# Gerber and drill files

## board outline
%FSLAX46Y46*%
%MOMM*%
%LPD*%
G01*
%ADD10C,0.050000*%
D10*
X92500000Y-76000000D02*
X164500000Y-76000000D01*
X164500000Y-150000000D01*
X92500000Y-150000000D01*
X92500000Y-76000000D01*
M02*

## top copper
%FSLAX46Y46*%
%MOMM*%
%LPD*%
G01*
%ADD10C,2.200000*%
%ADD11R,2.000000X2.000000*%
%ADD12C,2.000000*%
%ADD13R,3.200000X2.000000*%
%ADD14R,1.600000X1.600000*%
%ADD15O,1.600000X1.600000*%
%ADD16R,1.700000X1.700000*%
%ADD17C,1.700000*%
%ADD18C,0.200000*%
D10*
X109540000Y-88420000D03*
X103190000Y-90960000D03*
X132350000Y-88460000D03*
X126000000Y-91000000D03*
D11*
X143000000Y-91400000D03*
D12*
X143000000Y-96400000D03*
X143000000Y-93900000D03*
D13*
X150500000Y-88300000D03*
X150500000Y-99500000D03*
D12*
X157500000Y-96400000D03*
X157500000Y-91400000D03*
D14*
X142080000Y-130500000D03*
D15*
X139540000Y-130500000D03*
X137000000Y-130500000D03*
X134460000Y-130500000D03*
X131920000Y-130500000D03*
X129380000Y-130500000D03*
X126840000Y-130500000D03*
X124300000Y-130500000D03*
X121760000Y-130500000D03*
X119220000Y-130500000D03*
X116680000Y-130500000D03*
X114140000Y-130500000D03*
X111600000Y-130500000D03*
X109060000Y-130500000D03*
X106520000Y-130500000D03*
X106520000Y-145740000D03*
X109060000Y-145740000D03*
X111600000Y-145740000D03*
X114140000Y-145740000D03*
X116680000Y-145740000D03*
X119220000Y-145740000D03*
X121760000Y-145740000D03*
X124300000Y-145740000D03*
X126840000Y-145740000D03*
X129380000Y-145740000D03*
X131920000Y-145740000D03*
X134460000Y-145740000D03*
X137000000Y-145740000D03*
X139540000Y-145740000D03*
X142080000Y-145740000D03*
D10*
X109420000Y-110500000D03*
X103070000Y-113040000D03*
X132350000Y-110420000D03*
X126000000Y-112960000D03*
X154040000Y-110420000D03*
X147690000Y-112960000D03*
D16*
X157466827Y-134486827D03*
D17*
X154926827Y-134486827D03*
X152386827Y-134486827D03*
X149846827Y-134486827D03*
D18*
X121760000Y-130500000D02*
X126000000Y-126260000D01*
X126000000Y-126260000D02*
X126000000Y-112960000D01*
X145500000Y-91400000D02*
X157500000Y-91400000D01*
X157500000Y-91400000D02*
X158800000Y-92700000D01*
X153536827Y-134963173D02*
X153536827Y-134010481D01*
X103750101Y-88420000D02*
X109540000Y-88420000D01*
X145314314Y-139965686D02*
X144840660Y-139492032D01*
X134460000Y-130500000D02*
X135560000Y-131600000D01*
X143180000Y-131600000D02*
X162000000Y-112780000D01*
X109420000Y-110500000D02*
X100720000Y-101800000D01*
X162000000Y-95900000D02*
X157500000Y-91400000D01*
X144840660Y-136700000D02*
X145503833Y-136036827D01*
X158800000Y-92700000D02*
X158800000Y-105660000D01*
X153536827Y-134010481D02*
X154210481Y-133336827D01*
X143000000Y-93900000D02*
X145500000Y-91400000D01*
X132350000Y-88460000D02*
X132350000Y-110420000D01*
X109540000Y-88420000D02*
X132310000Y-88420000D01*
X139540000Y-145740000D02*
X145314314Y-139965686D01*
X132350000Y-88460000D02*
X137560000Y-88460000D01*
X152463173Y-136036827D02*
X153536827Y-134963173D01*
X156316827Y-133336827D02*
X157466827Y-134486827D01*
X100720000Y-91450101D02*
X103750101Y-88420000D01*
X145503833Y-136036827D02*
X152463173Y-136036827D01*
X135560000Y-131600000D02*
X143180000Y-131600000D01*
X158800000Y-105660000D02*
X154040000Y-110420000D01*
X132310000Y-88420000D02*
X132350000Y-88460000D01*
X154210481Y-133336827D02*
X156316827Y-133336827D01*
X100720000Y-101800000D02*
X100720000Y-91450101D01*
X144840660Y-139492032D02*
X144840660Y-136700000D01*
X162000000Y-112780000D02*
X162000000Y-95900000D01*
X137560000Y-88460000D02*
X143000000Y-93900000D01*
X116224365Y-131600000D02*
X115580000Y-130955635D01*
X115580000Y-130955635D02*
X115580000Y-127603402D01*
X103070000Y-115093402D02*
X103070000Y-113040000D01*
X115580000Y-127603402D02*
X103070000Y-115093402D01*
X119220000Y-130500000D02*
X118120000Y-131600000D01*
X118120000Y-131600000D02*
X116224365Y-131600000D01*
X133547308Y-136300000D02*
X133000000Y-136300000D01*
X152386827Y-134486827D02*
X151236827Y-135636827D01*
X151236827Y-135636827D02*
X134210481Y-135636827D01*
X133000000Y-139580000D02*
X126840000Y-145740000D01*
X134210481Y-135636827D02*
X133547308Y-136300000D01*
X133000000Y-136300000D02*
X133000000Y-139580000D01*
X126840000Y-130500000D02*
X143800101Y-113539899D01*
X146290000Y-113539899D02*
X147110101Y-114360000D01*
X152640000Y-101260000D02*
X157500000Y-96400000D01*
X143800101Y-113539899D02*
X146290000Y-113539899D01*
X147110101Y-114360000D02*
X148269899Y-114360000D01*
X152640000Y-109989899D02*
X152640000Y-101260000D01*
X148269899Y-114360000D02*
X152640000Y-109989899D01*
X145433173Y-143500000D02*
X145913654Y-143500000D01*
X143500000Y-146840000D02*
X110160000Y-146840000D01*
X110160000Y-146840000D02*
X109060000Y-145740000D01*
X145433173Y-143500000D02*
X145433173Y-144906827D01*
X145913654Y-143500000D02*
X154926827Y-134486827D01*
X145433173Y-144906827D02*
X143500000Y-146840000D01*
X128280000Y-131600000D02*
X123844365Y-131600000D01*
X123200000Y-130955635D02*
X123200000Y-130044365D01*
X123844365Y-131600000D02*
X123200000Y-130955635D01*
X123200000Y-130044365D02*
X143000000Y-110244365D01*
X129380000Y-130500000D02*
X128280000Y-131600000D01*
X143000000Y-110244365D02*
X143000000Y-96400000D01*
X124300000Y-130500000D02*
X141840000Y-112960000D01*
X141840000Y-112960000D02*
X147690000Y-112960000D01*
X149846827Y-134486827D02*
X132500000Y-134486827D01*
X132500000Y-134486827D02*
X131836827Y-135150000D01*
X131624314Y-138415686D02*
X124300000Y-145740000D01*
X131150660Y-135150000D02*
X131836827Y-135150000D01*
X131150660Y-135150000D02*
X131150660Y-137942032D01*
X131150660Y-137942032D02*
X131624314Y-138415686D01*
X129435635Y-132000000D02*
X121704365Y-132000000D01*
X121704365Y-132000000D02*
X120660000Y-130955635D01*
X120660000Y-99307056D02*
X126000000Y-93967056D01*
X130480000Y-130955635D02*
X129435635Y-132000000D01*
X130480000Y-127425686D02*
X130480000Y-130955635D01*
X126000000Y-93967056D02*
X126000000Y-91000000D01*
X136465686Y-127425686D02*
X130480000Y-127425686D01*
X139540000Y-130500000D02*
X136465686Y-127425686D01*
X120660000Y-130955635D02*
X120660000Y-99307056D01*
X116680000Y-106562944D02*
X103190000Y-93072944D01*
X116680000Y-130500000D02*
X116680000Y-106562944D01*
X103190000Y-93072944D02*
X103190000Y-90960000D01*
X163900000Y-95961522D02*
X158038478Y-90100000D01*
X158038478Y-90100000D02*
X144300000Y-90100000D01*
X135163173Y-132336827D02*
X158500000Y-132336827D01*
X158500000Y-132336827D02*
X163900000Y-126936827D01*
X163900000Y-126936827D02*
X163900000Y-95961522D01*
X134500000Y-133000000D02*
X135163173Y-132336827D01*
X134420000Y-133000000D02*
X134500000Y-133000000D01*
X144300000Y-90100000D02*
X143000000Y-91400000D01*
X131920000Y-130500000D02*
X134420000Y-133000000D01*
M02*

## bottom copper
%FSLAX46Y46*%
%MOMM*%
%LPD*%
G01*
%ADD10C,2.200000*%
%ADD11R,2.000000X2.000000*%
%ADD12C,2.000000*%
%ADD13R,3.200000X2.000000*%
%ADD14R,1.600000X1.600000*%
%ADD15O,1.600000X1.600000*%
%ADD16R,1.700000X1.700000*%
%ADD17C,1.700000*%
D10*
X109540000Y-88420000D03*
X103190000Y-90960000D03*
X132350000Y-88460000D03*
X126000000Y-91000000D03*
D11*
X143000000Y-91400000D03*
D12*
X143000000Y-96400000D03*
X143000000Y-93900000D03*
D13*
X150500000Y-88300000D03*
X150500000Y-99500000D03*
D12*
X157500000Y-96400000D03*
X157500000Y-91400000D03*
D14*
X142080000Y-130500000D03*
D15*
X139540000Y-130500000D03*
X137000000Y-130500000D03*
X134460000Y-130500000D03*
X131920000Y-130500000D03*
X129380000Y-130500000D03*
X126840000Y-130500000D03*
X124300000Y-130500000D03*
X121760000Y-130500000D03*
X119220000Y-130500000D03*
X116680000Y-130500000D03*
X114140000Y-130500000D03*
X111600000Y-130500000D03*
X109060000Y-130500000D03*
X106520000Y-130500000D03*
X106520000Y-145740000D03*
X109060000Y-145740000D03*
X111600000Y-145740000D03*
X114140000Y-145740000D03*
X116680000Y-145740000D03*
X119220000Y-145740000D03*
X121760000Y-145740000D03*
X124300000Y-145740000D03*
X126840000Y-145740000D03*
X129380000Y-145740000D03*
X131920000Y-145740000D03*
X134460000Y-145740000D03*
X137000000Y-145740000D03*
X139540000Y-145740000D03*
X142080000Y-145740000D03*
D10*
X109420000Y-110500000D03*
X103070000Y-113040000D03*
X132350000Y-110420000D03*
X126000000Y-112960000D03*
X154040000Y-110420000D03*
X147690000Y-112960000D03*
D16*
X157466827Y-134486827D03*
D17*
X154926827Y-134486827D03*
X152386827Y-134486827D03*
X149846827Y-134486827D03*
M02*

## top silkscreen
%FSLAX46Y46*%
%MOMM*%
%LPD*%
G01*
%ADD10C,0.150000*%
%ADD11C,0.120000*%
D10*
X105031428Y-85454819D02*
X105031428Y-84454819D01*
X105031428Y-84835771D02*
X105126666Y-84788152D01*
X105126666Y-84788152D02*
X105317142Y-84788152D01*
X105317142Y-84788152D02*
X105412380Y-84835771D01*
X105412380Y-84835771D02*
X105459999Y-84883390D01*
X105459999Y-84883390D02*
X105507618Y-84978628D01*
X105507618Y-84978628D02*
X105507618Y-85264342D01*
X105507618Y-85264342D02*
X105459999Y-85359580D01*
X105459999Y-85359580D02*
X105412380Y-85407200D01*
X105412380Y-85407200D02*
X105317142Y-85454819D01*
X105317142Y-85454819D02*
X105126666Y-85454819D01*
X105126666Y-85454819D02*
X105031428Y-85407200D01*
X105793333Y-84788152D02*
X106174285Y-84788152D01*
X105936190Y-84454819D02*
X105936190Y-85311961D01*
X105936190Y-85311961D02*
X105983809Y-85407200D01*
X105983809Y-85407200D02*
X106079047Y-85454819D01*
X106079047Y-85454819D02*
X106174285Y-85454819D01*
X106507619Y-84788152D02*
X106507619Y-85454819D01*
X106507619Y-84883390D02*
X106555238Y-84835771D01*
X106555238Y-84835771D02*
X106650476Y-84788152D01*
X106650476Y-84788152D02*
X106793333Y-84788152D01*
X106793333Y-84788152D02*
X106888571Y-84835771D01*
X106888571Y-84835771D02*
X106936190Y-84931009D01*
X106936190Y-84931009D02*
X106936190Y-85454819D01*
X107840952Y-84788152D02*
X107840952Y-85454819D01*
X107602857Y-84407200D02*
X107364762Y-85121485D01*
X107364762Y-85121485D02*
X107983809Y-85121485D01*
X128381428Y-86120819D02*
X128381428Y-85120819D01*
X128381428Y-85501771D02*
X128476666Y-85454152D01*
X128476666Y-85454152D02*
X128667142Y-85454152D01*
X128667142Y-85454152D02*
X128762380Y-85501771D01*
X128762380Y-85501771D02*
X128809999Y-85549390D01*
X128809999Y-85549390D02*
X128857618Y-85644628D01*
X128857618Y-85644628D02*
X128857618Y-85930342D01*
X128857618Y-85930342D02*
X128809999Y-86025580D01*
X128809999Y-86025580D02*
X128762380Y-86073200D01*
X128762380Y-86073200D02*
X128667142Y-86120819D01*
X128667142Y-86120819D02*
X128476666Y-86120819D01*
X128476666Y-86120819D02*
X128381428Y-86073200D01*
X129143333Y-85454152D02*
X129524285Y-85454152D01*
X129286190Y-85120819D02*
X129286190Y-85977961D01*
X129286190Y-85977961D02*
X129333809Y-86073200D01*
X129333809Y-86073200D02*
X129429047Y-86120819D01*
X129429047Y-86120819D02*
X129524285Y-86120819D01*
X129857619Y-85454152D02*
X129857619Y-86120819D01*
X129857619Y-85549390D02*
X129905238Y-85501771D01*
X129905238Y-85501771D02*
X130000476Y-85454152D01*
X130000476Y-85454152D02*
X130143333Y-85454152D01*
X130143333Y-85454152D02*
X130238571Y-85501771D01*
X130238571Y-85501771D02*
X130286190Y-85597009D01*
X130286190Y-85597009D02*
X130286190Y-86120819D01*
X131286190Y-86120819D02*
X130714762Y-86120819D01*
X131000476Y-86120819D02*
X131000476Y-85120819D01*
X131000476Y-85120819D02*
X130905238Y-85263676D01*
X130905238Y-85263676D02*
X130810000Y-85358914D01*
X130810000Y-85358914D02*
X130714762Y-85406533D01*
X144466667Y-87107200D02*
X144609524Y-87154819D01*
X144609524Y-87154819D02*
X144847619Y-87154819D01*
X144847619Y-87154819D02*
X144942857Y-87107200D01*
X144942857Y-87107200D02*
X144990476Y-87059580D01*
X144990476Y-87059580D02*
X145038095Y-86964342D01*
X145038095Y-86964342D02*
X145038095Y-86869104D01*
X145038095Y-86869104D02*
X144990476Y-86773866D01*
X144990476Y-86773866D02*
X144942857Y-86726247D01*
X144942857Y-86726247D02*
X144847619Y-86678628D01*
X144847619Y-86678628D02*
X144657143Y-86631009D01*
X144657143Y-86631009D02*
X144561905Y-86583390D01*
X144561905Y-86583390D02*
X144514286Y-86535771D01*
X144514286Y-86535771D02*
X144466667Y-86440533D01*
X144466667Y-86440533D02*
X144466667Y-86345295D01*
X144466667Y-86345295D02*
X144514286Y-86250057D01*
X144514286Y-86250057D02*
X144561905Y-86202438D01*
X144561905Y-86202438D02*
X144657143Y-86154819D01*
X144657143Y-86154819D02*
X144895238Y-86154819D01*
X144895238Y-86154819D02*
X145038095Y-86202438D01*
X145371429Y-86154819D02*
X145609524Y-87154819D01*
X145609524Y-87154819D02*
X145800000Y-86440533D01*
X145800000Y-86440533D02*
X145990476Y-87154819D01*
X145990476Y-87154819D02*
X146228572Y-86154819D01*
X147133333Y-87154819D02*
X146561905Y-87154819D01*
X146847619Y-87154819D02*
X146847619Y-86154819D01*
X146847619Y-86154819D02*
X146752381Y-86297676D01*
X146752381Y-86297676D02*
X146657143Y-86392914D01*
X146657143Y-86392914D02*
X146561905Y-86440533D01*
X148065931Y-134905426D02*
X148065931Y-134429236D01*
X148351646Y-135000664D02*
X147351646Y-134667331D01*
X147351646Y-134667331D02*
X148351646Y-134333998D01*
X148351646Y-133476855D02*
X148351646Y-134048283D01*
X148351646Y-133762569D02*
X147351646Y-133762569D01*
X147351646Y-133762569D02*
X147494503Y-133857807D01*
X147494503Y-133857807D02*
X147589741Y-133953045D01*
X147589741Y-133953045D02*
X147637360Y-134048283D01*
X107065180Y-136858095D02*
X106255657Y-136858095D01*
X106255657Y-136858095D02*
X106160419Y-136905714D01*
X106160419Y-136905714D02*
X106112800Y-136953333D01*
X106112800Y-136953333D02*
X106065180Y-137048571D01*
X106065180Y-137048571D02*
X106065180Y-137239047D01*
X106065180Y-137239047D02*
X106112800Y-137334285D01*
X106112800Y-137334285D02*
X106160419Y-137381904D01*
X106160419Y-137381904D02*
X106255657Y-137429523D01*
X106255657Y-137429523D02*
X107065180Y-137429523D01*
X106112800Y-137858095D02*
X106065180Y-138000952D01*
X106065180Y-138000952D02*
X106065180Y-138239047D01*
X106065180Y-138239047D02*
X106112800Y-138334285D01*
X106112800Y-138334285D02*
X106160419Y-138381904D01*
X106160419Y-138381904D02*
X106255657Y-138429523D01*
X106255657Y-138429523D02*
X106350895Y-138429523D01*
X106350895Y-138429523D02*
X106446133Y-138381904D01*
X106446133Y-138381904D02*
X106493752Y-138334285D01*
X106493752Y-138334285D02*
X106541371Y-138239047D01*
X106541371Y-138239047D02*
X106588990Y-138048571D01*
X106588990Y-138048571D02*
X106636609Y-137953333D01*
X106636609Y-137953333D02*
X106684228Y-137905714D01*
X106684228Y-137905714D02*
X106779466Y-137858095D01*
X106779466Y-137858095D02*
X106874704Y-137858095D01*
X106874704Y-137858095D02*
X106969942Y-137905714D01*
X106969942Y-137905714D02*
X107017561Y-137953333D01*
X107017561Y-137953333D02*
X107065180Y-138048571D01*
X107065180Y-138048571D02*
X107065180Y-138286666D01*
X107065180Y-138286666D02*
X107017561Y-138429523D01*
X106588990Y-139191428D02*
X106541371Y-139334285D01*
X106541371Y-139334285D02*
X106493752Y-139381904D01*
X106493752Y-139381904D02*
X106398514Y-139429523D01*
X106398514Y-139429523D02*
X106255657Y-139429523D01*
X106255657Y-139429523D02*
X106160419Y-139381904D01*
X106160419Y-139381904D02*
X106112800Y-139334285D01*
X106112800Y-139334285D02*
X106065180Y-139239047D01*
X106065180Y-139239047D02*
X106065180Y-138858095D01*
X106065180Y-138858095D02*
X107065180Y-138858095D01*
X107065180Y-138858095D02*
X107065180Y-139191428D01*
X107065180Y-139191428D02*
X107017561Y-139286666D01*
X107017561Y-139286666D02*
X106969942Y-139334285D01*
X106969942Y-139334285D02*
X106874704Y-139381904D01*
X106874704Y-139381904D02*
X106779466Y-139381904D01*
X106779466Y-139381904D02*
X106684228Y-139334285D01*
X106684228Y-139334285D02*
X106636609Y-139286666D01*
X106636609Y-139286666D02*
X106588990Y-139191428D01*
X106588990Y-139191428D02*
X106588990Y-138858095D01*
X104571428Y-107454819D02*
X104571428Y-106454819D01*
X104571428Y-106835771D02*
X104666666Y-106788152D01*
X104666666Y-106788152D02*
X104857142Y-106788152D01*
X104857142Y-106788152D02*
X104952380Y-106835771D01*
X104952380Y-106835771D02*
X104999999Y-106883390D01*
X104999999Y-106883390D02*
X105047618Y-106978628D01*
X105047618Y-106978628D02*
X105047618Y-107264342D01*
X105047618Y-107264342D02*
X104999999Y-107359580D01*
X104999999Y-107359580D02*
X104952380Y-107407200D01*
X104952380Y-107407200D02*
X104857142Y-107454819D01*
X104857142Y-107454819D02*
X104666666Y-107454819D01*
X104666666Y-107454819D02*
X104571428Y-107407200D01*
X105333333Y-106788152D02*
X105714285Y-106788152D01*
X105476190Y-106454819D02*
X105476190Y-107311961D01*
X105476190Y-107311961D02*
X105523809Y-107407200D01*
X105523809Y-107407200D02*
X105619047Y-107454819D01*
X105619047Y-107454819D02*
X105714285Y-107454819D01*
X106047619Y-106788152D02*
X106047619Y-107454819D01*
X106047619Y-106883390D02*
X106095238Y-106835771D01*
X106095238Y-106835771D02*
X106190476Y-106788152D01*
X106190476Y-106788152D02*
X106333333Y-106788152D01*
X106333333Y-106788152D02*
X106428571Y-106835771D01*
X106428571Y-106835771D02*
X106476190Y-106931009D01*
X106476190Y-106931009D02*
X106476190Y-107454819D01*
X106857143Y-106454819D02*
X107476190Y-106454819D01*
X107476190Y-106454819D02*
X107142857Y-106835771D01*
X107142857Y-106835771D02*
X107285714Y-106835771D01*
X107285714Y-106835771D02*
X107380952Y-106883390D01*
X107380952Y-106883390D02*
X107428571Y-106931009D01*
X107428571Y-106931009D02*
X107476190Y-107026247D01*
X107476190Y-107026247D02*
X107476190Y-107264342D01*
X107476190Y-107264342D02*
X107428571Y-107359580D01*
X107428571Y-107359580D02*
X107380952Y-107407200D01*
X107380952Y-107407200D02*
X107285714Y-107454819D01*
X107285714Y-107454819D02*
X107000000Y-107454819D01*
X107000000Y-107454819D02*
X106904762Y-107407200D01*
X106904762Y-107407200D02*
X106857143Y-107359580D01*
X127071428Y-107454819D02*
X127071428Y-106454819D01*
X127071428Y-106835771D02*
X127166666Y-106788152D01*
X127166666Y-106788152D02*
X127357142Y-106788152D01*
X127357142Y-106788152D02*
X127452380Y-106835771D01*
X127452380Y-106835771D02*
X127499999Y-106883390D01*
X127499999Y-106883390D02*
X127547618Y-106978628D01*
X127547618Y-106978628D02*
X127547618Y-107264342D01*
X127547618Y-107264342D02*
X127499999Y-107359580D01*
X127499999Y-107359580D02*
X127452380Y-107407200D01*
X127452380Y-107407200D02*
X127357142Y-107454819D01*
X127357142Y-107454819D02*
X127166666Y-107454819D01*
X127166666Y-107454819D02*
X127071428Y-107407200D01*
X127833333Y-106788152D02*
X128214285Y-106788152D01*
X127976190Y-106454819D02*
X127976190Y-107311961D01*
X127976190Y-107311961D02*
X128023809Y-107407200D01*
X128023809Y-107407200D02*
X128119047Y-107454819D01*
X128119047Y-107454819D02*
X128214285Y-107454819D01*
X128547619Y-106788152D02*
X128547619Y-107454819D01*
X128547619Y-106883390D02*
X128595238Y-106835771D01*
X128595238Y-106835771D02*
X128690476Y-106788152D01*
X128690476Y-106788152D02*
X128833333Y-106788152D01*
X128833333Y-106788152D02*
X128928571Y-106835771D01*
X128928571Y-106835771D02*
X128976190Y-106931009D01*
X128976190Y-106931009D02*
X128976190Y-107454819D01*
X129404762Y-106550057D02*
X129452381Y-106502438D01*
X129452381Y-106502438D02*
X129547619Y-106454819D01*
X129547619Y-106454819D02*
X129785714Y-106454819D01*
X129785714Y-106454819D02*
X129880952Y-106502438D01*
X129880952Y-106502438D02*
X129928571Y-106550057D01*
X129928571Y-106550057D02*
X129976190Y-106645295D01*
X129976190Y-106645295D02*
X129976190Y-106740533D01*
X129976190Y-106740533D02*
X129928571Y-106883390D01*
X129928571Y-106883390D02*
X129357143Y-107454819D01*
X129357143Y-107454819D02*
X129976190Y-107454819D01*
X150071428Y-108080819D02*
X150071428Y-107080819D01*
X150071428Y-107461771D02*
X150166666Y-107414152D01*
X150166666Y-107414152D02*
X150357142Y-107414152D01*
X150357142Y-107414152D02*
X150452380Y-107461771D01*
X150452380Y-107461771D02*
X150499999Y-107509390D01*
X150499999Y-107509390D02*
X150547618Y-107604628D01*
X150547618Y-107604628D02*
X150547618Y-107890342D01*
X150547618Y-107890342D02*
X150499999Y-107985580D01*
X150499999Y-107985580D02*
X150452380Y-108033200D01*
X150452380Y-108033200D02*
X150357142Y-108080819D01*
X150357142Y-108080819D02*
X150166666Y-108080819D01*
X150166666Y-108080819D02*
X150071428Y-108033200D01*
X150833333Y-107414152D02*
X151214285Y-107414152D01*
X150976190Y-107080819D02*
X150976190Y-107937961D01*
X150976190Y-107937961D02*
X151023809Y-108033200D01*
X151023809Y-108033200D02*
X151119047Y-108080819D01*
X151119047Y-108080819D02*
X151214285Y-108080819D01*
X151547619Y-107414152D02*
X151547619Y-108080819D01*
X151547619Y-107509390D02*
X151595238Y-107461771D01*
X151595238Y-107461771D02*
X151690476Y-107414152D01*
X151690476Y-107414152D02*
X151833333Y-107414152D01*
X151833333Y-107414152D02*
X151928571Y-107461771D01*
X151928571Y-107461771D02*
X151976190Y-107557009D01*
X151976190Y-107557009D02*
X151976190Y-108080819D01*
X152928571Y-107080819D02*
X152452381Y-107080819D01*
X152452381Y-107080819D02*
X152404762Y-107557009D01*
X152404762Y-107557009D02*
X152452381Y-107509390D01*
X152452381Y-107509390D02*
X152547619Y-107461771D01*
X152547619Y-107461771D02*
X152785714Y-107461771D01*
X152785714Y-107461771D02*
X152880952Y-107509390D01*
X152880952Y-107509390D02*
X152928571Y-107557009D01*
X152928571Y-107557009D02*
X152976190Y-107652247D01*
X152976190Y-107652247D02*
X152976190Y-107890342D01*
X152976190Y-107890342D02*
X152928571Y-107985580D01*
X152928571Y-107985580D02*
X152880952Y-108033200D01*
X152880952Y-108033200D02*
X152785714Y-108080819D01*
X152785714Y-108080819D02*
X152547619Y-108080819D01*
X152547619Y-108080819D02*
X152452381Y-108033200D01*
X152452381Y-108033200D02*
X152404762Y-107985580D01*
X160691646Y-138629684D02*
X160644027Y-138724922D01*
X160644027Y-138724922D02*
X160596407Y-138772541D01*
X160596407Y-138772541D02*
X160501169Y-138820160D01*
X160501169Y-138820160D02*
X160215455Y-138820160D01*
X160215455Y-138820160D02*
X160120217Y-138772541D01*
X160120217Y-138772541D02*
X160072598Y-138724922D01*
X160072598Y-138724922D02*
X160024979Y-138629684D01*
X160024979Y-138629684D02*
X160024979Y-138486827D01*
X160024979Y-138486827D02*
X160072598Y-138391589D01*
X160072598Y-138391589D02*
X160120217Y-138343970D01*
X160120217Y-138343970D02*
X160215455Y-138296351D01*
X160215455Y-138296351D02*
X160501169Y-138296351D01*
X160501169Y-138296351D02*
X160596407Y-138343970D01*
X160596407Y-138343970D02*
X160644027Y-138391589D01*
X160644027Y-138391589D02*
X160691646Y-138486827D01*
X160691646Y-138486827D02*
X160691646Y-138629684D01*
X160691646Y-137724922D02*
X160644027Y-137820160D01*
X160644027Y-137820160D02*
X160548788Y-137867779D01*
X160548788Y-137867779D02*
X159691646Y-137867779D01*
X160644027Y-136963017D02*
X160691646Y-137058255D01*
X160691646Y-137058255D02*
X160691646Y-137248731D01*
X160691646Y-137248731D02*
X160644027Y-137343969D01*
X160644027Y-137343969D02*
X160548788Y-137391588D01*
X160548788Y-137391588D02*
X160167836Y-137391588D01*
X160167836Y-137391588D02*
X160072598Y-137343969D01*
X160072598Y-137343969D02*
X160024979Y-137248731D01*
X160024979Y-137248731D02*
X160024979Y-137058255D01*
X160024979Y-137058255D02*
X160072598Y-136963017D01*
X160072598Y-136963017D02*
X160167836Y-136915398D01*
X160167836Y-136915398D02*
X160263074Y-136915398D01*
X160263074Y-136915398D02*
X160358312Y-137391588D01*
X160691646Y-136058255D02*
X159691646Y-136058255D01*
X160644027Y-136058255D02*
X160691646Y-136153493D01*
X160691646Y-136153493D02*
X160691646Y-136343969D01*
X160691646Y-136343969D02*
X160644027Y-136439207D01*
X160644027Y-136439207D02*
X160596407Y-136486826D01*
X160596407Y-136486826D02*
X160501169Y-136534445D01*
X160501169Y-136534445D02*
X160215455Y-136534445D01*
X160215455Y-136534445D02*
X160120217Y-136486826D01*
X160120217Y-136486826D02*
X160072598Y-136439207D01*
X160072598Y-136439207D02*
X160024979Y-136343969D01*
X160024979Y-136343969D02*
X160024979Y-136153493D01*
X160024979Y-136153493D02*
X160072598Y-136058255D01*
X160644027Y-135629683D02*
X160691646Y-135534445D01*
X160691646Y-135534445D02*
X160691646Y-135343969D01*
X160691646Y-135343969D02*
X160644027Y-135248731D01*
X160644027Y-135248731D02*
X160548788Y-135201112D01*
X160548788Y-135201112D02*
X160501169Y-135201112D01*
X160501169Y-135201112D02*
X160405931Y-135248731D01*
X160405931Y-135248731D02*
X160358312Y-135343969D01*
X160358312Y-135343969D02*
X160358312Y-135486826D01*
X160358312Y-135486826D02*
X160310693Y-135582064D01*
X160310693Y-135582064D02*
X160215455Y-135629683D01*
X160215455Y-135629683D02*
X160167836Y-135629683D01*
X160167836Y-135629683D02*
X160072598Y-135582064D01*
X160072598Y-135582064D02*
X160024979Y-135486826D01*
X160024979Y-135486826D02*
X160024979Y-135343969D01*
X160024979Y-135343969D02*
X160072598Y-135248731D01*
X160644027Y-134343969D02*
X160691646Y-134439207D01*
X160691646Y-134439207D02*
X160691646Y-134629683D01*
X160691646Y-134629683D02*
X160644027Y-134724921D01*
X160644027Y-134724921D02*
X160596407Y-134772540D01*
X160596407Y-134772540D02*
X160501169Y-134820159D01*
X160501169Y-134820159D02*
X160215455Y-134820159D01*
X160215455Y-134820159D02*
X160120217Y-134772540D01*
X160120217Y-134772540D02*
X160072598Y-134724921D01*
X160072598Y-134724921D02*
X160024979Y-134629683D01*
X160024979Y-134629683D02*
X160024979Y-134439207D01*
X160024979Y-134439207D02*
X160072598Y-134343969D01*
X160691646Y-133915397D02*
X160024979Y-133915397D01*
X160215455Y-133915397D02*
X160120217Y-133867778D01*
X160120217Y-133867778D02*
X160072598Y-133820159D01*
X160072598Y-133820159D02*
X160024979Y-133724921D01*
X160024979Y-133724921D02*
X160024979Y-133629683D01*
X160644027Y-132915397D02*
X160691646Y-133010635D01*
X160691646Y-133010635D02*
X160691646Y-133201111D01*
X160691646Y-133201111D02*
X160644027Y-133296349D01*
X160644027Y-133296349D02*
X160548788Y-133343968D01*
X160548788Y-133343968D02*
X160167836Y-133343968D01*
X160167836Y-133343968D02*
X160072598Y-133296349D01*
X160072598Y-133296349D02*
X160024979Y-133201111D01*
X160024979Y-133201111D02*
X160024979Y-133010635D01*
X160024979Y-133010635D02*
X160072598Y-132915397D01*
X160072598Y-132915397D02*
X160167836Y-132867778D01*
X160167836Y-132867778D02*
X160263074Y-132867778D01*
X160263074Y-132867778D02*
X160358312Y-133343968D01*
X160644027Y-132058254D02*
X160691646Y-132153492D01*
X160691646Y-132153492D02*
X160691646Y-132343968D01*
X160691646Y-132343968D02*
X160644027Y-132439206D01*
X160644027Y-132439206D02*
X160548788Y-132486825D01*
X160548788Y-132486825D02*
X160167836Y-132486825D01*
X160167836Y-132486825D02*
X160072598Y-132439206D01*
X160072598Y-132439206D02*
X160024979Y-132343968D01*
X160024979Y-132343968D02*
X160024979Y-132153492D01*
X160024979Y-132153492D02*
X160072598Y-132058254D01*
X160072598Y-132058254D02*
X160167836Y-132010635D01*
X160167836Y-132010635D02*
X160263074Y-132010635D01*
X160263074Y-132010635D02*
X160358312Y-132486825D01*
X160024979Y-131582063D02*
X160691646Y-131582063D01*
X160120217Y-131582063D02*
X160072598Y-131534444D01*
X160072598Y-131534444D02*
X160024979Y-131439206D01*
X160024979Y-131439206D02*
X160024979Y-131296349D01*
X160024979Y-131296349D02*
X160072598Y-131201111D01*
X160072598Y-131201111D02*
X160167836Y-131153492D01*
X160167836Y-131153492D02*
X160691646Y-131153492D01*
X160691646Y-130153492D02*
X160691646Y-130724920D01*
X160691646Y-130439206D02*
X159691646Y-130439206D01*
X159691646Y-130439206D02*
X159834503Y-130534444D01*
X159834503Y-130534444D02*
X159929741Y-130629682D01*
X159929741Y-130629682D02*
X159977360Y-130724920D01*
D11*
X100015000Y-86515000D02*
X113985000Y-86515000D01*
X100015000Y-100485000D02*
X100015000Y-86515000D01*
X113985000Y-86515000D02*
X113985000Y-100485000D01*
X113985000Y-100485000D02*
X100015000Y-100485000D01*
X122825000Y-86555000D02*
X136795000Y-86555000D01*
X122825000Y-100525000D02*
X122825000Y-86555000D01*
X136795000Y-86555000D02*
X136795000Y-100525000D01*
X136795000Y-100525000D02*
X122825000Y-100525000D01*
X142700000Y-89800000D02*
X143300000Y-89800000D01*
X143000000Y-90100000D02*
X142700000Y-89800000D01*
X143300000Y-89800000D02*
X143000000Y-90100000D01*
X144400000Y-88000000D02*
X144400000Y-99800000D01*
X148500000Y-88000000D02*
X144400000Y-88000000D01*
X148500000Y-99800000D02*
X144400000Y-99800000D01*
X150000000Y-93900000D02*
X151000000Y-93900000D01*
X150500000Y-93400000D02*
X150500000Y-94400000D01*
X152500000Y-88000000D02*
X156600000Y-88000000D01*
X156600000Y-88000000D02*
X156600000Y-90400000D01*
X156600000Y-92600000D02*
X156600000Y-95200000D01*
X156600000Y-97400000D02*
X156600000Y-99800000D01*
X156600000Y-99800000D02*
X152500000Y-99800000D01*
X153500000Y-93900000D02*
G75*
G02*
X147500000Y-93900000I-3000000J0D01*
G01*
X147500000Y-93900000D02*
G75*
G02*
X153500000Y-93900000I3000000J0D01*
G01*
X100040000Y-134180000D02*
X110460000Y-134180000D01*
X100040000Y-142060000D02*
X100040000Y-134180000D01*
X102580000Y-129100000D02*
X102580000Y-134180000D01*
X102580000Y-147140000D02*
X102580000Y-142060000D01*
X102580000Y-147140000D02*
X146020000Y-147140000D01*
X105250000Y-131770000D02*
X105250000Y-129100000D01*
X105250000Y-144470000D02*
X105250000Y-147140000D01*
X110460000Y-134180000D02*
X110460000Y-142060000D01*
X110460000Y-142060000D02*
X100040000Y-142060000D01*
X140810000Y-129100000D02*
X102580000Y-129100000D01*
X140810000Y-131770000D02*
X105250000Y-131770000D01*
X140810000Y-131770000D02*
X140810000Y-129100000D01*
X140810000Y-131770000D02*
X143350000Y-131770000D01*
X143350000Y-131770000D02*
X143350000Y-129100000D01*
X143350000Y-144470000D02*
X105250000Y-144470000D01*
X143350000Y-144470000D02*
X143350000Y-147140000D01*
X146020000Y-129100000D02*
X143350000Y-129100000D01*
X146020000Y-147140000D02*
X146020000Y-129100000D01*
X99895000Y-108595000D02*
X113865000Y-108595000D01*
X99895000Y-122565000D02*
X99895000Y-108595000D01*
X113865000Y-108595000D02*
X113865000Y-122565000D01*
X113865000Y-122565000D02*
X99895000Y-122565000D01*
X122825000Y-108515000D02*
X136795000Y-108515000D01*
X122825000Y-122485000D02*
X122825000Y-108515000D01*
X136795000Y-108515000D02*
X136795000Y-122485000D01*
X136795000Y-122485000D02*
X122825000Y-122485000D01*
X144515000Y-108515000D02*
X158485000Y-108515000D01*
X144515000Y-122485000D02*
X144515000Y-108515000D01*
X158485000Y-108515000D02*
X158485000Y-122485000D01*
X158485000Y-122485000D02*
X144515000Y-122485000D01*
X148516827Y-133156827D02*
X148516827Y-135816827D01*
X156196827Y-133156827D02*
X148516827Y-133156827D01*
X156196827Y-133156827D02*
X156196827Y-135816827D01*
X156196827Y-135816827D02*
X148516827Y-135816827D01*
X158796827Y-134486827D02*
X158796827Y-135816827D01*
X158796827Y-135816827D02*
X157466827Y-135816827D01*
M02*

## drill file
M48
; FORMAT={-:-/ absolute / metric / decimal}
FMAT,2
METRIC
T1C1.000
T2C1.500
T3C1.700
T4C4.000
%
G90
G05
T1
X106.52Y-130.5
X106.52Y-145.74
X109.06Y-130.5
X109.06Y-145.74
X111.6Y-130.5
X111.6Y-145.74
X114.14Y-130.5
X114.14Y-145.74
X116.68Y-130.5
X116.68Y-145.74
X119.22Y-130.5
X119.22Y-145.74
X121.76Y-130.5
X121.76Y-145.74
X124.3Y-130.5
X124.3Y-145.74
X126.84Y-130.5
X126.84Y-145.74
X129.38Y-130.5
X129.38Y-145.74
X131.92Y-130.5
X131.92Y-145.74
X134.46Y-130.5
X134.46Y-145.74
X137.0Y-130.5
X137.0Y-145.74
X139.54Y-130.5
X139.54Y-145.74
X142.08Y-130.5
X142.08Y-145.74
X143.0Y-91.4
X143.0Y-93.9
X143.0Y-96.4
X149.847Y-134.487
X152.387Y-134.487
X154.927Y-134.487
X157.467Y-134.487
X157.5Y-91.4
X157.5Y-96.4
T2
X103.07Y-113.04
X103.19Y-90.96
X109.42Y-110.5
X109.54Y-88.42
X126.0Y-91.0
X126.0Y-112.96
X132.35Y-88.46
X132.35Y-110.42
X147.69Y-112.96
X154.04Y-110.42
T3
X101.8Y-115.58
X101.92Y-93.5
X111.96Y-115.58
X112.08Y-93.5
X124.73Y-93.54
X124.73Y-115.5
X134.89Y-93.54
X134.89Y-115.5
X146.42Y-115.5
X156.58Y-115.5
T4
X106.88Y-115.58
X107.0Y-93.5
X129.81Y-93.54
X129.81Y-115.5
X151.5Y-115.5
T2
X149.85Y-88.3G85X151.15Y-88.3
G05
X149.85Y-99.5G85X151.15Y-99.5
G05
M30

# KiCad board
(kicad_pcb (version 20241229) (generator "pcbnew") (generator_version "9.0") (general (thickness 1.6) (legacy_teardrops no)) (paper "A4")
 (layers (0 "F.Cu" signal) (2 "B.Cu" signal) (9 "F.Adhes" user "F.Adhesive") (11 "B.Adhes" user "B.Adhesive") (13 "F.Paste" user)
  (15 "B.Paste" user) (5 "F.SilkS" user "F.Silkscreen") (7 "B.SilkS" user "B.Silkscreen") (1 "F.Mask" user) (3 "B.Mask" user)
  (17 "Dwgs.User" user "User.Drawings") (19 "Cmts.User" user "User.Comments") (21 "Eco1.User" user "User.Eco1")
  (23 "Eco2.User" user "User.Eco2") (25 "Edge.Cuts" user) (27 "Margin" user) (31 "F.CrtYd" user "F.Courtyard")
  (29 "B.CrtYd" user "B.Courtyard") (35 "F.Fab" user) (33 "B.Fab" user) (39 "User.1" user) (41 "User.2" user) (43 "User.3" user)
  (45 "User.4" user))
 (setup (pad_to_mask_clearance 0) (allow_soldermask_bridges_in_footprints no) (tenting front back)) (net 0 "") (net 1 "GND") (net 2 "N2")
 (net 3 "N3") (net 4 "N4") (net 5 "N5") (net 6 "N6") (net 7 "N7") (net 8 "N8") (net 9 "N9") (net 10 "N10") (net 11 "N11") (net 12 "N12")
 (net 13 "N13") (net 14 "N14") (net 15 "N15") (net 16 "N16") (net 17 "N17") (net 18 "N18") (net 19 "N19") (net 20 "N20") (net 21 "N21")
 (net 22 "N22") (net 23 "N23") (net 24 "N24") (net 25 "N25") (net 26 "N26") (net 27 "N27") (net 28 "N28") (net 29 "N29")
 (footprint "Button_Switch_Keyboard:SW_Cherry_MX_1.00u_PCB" (layer "F.Cu") (at 109.54 88.42)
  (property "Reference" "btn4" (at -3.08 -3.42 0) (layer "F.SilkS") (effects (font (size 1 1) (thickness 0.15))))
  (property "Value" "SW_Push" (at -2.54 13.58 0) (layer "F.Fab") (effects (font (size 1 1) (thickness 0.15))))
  (fp_line (start -9.525 -1.905) (end 4.445 -1.905) (stroke (width 0.12) (type solid)) (layer "F.SilkS"))
  (fp_line (start -9.525 12.065) (end -9.525 -1.905) (stroke (width 0.12) (type solid)) (layer "F.SilkS"))
  (fp_line (start 4.445 -1.905) (end 4.445 12.065) (stroke (width 0.12) (type solid)) (layer "F.SilkS"))
  (fp_line (start 4.445 12.065) (end -9.525 12.065) (stroke (width 0.12) (type solid)) (layer "F.SilkS"))
  (pad "" np_thru_hole circle (at -7.62 5.08) (size 1.7 1.7) (drill 1.7) (layers "*.Cu" "*.Mask"))
  (pad "" np_thru_hole circle (at -2.54 5.08) (size 4 4) (drill 4) (layers "*.Cu" "*.Mask"))
  (pad "" np_thru_hole circle (at 2.54 5.08) (size 1.7 1.7) (drill 1.7) (layers "*.Cu" "*.Mask"))
  (pad "1" thru_hole circle (at 0 0) (size 2.2 2.2) (drill 1.5) (layers "*.Cu" "*.Mask") (remove_unused_layers no) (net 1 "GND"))
  (pad "2" thru_hole circle (at -6.35 2.54) (size 2.2 2.2) (drill 1.5) (layers "*.Cu" "*.Mask") (remove_unused_layers no) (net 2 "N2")))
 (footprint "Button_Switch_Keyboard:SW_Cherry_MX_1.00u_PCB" (layer "F.Cu") (at 132.35 88.46)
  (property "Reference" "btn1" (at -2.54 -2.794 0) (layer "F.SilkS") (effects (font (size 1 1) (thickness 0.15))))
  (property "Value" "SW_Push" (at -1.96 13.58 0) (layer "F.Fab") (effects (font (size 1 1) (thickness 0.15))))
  (fp_line (start -9.525 -1.905) (end 4.445 -1.905) (stroke (width 0.12) (type solid)) (layer "F.SilkS"))
  (fp_line (start -9.525 12.065) (end -9.525 -1.905) (stroke (width 0.12) (type solid)) (layer "F.SilkS"))
  (fp_line (start 4.445 -1.905) (end 4.445 12.065) (stroke (width 0.12) (type solid)) (layer "F.SilkS"))
  (fp_line (start 4.445 12.065) (end -9.525 12.065) (stroke (width 0.12) (type solid)) (layer "F.SilkS"))
  (pad "" np_thru_hole circle (at -7.62 5.08) (size 1.7 1.7) (drill 1.7) (layers "*.Cu" "*.Mask"))
  (pad "" np_thru_hole circle (at -2.54 5.08) (size 4 4) (drill 4) (layers "*.Cu" "*.Mask"))
  (pad "" np_thru_hole circle (at 2.54 5.08) (size 1.7 1.7) (drill 1.7) (layers "*.Cu" "*.Mask"))
  (pad "1" thru_hole circle (at 0 0) (size 2.2 2.2) (drill 1.5) (layers "*.Cu" "*.Mask") (remove_unused_layers no) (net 1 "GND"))
  (pad "2" thru_hole circle (at -6.35 2.54) (size 2.2 2.2) (drill 1.5) (layers "*.Cu" "*.Mask") (remove_unused_layers no) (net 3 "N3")))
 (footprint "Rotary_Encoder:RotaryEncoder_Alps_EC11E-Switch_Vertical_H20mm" (layer "F.Cu") (at 143 91.4)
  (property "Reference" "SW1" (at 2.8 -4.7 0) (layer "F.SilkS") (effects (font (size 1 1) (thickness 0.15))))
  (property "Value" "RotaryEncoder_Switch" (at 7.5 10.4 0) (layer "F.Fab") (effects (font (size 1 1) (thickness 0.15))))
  (fp_line (start -0.3 -1.6) (end 0.3 -1.6) (stroke (width 0.12) (type solid)) (layer "F.SilkS"))
  (fp_line (start 0 -1.3) (end -0.3 -1.6) (stroke (width 0.12) (type solid)) (layer "F.SilkS"))
  (fp_line (start 0.3 -1.6) (end 0 -1.3) (stroke (width 0.12) (type solid)) (layer "F.SilkS"))
  (fp_line (start 1.4 -3.4) (end 1.4 8.4) (stroke (width 0.12) (type solid)) (layer "F.SilkS"))
  (fp_line (start 5.5 -3.4) (end 1.4 -3.4) (stroke (width 0.12) (type solid)) (layer "F.SilkS"))
  (fp_line (start 5.5 8.4) (end 1.4 8.4) (stroke (width 0.12) (type solid)) (layer "F.SilkS"))
  (fp_line (start 7 2.5) (end 8 2.5) (stroke (width 0.12) (type solid)) (layer "F.SilkS"))
  (fp_line (start 7.5 2) (end 7.5 3) (stroke (width 0.12) (type solid)) (layer "F.SilkS"))
  (fp_line (start 9.5 -3.4) (end 13.6 -3.4) (stroke (width 0.12) (type solid)) (layer "F.SilkS"))
  (fp_line (start 13.6 -3.4) (end 13.6 -1) (stroke (width 0.12) (type solid)) (layer "F.SilkS"))
  (fp_line (start 13.6 1.2) (end 13.6 3.8) (stroke (width 0.12) (type solid)) (layer "F.SilkS"))
  (fp_line (start 13.6 6) (end 13.6 8.4) (stroke (width 0.12) (type solid)) (layer "F.SilkS"))
  (fp_line (start 13.6 8.4) (end 9.5 8.4) (stroke (width 0.12) (type solid)) (layer "F.SilkS"))
  (fp_circle (center 7.5 2.5) (end 10.5 2.5) (stroke (width 0.12) (type solid)) (fill no) (layer "F.SilkS"))
  (pad "A" thru_hole rect (at 0 0) (size 2 2) (drill 1) (layers "*.Cu" "*.Mask") (remove_unused_layers no) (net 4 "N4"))
  (pad "B" thru_hole circle (at 0 5) (size 2 2) (drill 1) (layers "*.Cu" "*.Mask") (remove_unused_layers no) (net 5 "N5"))
  (pad "C" thru_hole circle (at 0 2.5) (size 2 2) (drill 1) (layers "*.Cu" "*.Mask") (remove_unused_layers no) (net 1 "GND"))
  (pad "MP" thru_hole rect (at 7.5 -3.1) (size 3.2 2) (drill oval 2.8 1.5) (layers "*.Cu" "*.Mask") (remove_unused_layers no))
  (pad "MP" thru_hole rect (at 7.5 8.1) (size 3.2 2) (drill oval 2.8 1.5) (layers "*.Cu" "*.Mask") (remove_unused_layers no))
  (pad "S1" thru_hole circle (at 14.5 5) (size 2 2) (drill 1) (layers "*.Cu" "*.Mask") (remove_unused_layers no) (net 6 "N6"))
  (pad "S2" thru_hole circle (at 14.5 0) (size 2 2) (drill 1) (layers "*.Cu" "*.Mask") (remove_unused_layers no) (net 1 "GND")))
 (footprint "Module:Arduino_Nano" (layer "F.Cu") (at 142.08 130.5 -90)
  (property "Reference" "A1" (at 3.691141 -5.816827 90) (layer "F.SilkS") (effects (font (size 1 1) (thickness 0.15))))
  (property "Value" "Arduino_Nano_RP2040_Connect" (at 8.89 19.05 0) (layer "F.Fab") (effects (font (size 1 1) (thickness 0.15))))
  (fp_line (start 3.68 42.04) (end 3.68 31.62) (stroke (width 0.12) (type solid)) (layer "F.SilkS"))
  (fp_line (start 11.56 42.04) (end 3.68 42.04) (stroke (width 0.12) (type solid)) (layer "F.SilkS"))
  (fp_line (start -1.4 39.5) (end 3.68 39.5) (stroke (width 0.12) (type solid)) (layer "F.SilkS"))
  (fp_line (start 16.64 39.5) (end 11.56 39.5) (stroke (width 0.12) (type solid)) (layer "F.SilkS"))
  (fp_line (start 16.64 39.5) (end 16.64 -3.94) (stroke (width 0.12) (type solid)) (layer "F.SilkS"))
  (fp_line (start 1.27 36.83) (end -1.4 36.83) (stroke (width 0.12) (type solid)) (layer "F.SilkS"))
  (fp_line (start 13.97 36.83) (end 16.64 36.83) (stroke (width 0.12) (type solid)) (layer "F.SilkS"))
  (fp_line (start 3.68 31.62) (end 11.56 31.62) (stroke (width 0.12) (type solid)) (layer "F.SilkS"))
  (fp_line (start 11.56 31.62) (end 11.56 42.04) (stroke (width 0.12) (type solid)) (layer "F.SilkS"))
  (fp_line (start -1.4 1.27) (end -1.4 39.5) (stroke (width 0.12) (type solid)) (layer "F.SilkS"))
  (fp_line (start 1.27 1.27) (end 1.27 36.83) (stroke (width 0.12) (type solid)) (layer "F.SilkS"))
  (fp_line (start 1.27 1.27) (end -1.4 1.27) (stroke (width 0.12) (type solid)) (layer "F.SilkS"))
  (fp_line (start 1.27 1.27) (end 1.27 -1.27) (stroke (width 0.12) (type solid)) (layer "F.SilkS"))
  (fp_line (start 1.27 -1.27) (end -1.4 -1.27) (stroke (width 0.12) (type solid)) (layer "F.SilkS"))
  (fp_line (start 13.97 -1.27) (end 13.97 36.83) (stroke (width 0.12) (type solid)) (layer "F.SilkS"))
  (fp_line (start 13.97 -1.27) (end 16.64 -1.27) (stroke (width 0.12) (type solid)) (layer "F.SilkS"))
  (fp_line (start -1.4 -3.94) (end -1.4 -1.27) (stroke (width 0.12) (type solid)) (layer "F.SilkS"))
  (fp_line (start 16.64 -3.94) (end -1.4 -3.94) (stroke (width 0.12) (type solid)) (layer "F.SilkS"))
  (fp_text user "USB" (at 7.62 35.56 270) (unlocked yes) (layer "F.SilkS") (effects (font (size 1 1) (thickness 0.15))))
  (pad "1" thru_hole rect (at 0 0 270) (size 1.6 1.6) (drill 1) (layers "*.Cu" "*.Mask") (remove_unused_layers no) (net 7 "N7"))
  (pad "2" thru_hole oval (at 0 2.54 270) (size 1.6 1.6) (drill 1) (layers "*.Cu" "*.Mask") (remove_unused_layers no) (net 3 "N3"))
  (pad "3" thru_hole oval (at 0 5.08 270) (size 1.6 1.6) (drill 1) (layers "*.Cu" "*.Mask") (remove_unused_layers no) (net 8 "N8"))
  (pad "4" thru_hole oval (at 0 7.62 270) (size 1.6 1.6) (drill 1) (layers "*.Cu" "*.Mask") (remove_unused_layers no) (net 1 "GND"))
  (pad "5" thru_hole oval (at 0 10.16 270) (size 1.6 1.6) (drill 1) (layers "*.Cu" "*.Mask") (remove_unused_layers no) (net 4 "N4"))
  (pad "6" thru_hole oval (at 0 12.7 270) (size 1.6 1.6) (drill 1) (layers "*.Cu" "*.Mask") (remove_unused_layers no) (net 5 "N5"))
  (pad "7" thru_hole oval (at 0 15.24 270) (size 1.6 1.6) (drill 1) (layers "*.Cu" "*.Mask") (remove_unused_layers no) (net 6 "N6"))
  (pad "8" thru_hole oval (at 0 17.78 270) (size 1.6 1.6) (drill 1) (layers "*.Cu" "*.Mask") (remove_unused_layers no) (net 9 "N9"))
  (pad "9" thru_hole oval (at 0 20.32 270) (size 1.6 1.6) (drill 1) (layers "*.Cu" "*.Mask") (remove_unused_layers no) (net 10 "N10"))
  (pad "10" thru_hole oval (at 0 22.86 270) (size 1.6 1.6) (drill 1) (layers "*.Cu" "*.Mask") (remove_unused_layers no) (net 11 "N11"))
  (pad "11" thru_hole oval (at 0 25.4 270) (size 1.6 1.6) (drill 1) (layers "*.Cu" "*.Mask") (remove_unused_layers no) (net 2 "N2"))
  (pad "12" thru_hole oval (at 0 27.94 270) (size 1.6 1.6) (drill 1) (layers "*.Cu" "*.Mask") (remove_unused_layers no) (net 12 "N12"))
  (pad "13" thru_hole oval (at 0 30.48 270) (size 1.6 1.6) (drill 1) (layers "*.Cu" "*.Mask") (remove_unused_layers no) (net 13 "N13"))
  (pad "14" thru_hole oval (at 0 33.02 270) (size 1.6 1.6) (drill 1) (layers "*.Cu" "*.Mask") (remove_unused_layers no) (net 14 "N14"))
  (pad "15" thru_hole oval (at 0 35.56 270) (size 1.6 1.6) (drill 1) (layers "*.Cu" "*.Mask") (remove_unused_layers no) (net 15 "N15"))
  (pad "16" thru_hole oval (at 15.24 35.56 270) (size 1.6 1.6) (drill 1) (layers "*.Cu" "*.Mask") (remove_unused_layers no) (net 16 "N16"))
  (pad "17" thru_hole oval (at 15.24 33.02 270) (size 1.6 1.6) (drill 1) (layers "*.Cu" "*.Mask") (remove_unused_layers no) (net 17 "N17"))
  (pad "18" thru_hole oval (at 15.24 30.48 270) (size 1.6 1.6) (drill 1) (layers "*.Cu" "*.Mask") (remove_unused_layers no) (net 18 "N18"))
  (pad "19" thru_hole oval (at 15.24 27.94 270) (size 1.6 1.6) (drill 1) (layers "*.Cu" "*.Mask") (remove_unused_layers no) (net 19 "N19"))
  (pad "20" thru_hole oval (at 15.24 25.4 270) (size 1.6 1.6) (drill 1) (layers "*.Cu" "*.Mask") (remove_unused_layers no) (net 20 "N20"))
  (pad "21" thru_hole oval (at 15.24 22.86 270) (size 1.6 1.6) (drill 1) (layers "*.Cu" "*.Mask") (remove_unused_layers no) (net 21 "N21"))
  (pad "22" thru_hole oval (at 15.24 20.32 270) (size 1.6 1.6) (drill 1) (layers "*.Cu" "*.Mask") (remove_unused_layers no) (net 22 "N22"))
  (pad "23" thru_hole oval (at 15.24 17.78 270) (size 1.6 1.6) (drill 1) (layers "*.Cu" "*.Mask") (remove_unused_layers no) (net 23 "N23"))
  (pad "24" thru_hole oval (at 15.24 15.24 270) (size 1.6 1.6) (drill 1) (layers "*.Cu" "*.Mask") (remove_unused_layers no) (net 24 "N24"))
  (pad "25" thru_hole oval (at 15.24 12.7 270) (size 1.6 1.6) (drill 1) (layers "*.Cu" "*.Mask") (remove_unused_layers no) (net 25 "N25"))
  (pad "26" thru_hole oval (at 15.24 10.16 270) (size 1.6 1.6) (drill 1) (layers "*.Cu" "*.Mask") (remove_unused_layers no) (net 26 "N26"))
  (pad "27" thru_hole oval (at 15.24 7.62 270) (size 1.6 1.6) (drill 1) (layers "*.Cu" "*.Mask") (remove_unused_layers no) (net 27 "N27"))
  (pad "28" thru_hole oval (at 15.24 5.08 270) (size 1.6 1.6) (drill 1) (layers "*.Cu" "*.Mask") (remove_unused_layers no) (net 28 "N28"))
  (pad "29" thru_hole oval (at 15.24 2.54 270) (size 1.6 1.6) (drill 1) (layers "*.Cu" "*.Mask") (remove_unused_layers no) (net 1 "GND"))
  (pad "30" thru_hole oval (at 15.24 0 270) (size 1.6 1.6) (drill 1) (layers "*.Cu" "*.Mask") (remove_unused_layers no) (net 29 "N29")))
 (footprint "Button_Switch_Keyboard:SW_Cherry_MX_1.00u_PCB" (layer "F.Cu") (at 109.42 110.5)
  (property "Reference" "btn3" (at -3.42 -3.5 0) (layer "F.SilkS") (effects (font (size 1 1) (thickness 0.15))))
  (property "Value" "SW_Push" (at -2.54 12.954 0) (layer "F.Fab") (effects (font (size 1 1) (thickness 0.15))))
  (fp_line (start -9.525 -1.905) (end 4.445 -1.905) (stroke (width 0.12) (type solid)) (layer "F.SilkS"))
  (fp_line (start -9.525 12.065) (end -9.525 -1.905) (stroke (width 0.12) (type solid)) (layer "F.SilkS"))
  (fp_line (start 4.445 -1.905) (end 4.445 12.065) (stroke (width 0.12) (type solid)) (layer "F.SilkS"))
  (fp_line (start 4.445 12.065) (end -9.525 12.065) (stroke (width 0.12) (type solid)) (layer "F.SilkS"))
  (pad "" np_thru_hole circle (at -7.62 5.08) (size 1.7 1.7) (drill 1.7) (layers "*.Cu" "*.Mask"))
  (pad "" np_thru_hole circle (at -2.54 5.08) (size 4 4) (drill 4) (layers "*.Cu" "*.Mask"))
  (pad "" np_thru_hole circle (at 2.54 5.08) (size 1.7 1.7) (drill 1.7) (layers "*.Cu" "*.Mask"))
  (pad "1" thru_hole circle (at 0 0) (size 2.2 2.2) (drill 1.5) (layers "*.Cu" "*.Mask") (remove_unused_layers no) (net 1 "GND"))
  (pad "2" thru_hole circle (at -6.35 2.54) (size 2.2 2.2) (drill 1.5) (layers "*.Cu" "*.Mask") (remove_unused_layers no) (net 11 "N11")))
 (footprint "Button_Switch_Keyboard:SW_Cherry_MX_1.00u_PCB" (layer "F.Cu") (at 132.35 110.42)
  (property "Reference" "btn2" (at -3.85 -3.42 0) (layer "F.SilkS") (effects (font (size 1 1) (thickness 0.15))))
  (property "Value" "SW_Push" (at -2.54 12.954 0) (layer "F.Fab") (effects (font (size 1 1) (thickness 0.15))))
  (fp_line (start -9.525 -1.905) (end 4.445 -1.905) (stroke (width 0.12) (type solid)) (layer "F.SilkS"))
  (fp_line (start -9.525 12.065) (end -9.525 -1.905) (stroke (width 0.12) (type solid)) (layer "F.SilkS"))
  (fp_line (start 4.445 -1.905) (end 4.445 12.065) (stroke (width 0.12) (type solid)) (layer "F.SilkS"))
  (fp_line (start 4.445 12.065) (end -9.525 12.065) (stroke (width 0.12) (type solid)) (layer "F.SilkS"))
  (pad "" np_thru_hole circle (at -7.62 5.08) (size 1.7 1.7) (drill 1.7) (layers "*.Cu" "*.Mask"))
  (pad "" np_thru_hole circle (at -2.54 5.08) (size 4 4) (drill 4) (layers "*.Cu" "*.Mask"))
  (pad "" np_thru_hole circle (at 2.54 5.08) (size 1.7 1.7) (drill 1.7) (layers "*.Cu" "*.Mask"))
  (pad "1" thru_hole circle (at 0 0) (size 2.2 2.2) (drill 1.5) (layers "*.Cu" "*.Mask") (remove_unused_layers no) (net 1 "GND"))
  (pad "2" thru_hole circle (at -6.35 2.54) (size 2.2 2.2) (drill 1.5) (layers "*.Cu" "*.Mask") (remove_unused_layers no) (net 10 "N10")))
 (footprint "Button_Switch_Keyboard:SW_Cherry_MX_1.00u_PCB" (layer "F.Cu") (at 154.04 110.42)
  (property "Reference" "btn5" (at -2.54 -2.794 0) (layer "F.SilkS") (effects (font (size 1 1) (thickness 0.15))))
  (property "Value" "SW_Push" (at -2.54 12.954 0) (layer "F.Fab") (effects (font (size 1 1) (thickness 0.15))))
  (fp_line (start -9.525 -1.905) (end 4.445 -1.905) (stroke (width 0.12) (type solid)) (layer "F.SilkS"))
  (fp_line (start -9.525 12.065) (end -9.525 -1.905) (stroke (width 0.12) (type solid)) (layer "F.SilkS"))
  (fp_line (start 4.445 -1.905) (end 4.445 12.065) (stroke (width 0.12) (type solid)) (layer "F.SilkS"))
  (fp_line (start 4.445 12.065) (end -9.525 12.065) (stroke (width 0.12) (type solid)) (layer "F.SilkS"))
  (pad "" np_thru_hole circle (at -7.62 5.08) (size 1.7 1.7) (drill 1.7) (layers "*.Cu" "*.Mask"))
  (pad "" np_thru_hole circle (at -2.54 5.08) (size 4 4) (drill 4) (layers "*.Cu" "*.Mask"))
  (pad "" np_thru_hole circle (at 2.54 5.08) (size 1.7 1.7) (drill 1.7) (layers "*.Cu" "*.Mask"))
  (pad "1" thru_hole circle (at 0 0) (size 2.2 2.2) (drill 1.5) (layers "*.Cu" "*.Mask") (remove_unused_layers no) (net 1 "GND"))
  (pad "2" thru_hole circle (at -6.35 2.54) (size 2.2 2.2) (drill 1.5) (layers "*.Cu" "*.Mask") (remove_unused_layers no) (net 9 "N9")))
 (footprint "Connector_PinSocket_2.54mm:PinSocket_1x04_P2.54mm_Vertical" (layer "F.Cu") (at 157.466827 134.486827 -90)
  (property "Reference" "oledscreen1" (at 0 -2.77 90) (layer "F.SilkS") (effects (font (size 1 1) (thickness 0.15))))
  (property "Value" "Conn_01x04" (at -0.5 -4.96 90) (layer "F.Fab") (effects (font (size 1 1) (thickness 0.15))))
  (fp_line (start -1.33 8.95) (end 1.33 8.95) (stroke (width 0.12) (type solid)) (layer "F.SilkS"))
  (fp_line (start -1.33 1.27) (end -1.33 8.95) (stroke (width 0.12) (type solid)) (layer "F.SilkS"))
  (fp_line (start -1.33 1.27) (end 1.33 1.27) (stroke (width 0.12) (type solid)) (layer "F.SilkS"))
  (fp_line (start 1.33 1.27) (end 1.33 8.95) (stroke (width 0.12) (type solid)) (layer "F.SilkS"))
  (fp_line (start 0 -1.33) (end 1.33 -1.33) (stroke (width 0.12) (type solid)) (layer "F.SilkS"))
  (fp_line (start 1.33 -1.33) (end 1.33 0) (stroke (width 0.12) (type solid)) (layer "F.SilkS"))
  (pad "1" thru_hole rect (at 0 0 270) (size 1.7 1.7) (drill 1) (layers "*.Cu" "*.Mask") (remove_unused_layers no) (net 1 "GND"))
  (pad "2" thru_hole circle (at 0 2.54 270) (size 1.7 1.7) (drill 1) (layers "*.Cu" "*.Mask") (remove_unused_layers no) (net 17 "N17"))
  (pad "3" thru_hole circle (at 0 5.08 270) (size 1.7 1.7) (drill 1) (layers "*.Cu" "*.Mask") (remove_unused_layers no) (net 24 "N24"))
  (pad "4" thru_hole circle (at 0 7.62 270) (size 1.7 1.7) (drill 1) (layers "*.Cu" "*.Mask") (remove_unused_layers no) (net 23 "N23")))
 (gr_rect (start 92.5 76) (end 164.5 150) (stroke (width 0.05) (type default)) (fill no) (layer "Edge.Cuts"))
 (segment (start 121.76 130.5) (end 126 126.26) (width 0.2) (layer "F.Cu") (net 10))
 (segment (start 126 126.26) (end 126 112.96) (width 0.2) (layer "F.Cu") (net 10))
 (segment (start 145.5 91.4) (end 157.5 91.4) (width 0.2) (layer "F.Cu") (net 1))
 (segment (start 157.5 91.4) (end 158.8 92.7) (width 0.2) (layer "F.Cu") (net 1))
 (segment (start 153.536827 134.963173) (end 153.536827 134.010481) (width 0.2) (layer "F.Cu") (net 1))
 (segment (start 103.750101 88.42) (end 109.54 88.42) (width 0.2) (layer "F.Cu") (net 1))
 (segment (start 145.314314 139.965686) (end 144.84066 139.492032) (width 0.2) (layer "F.Cu") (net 1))
 (segment (start 134.46 130.5) (end 135.56 131.6) (width 0.2) (layer "F.Cu") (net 1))
 (segment (start 143.18 131.6) (end 162 112.78) (width 0.2) (layer "F.Cu") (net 1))
 (segment (start 109.42 110.5) (end 100.72 101.8) (width 0.2) (layer "F.Cu") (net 1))
 (segment (start 162 95.9) (end 157.5 91.4) (width 0.2) (layer "F.Cu") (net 1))
 (segment (start 144.84066 136.7) (end 145.503833 136.036827) (width 0.2) (layer "F.Cu") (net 1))
 (segment (start 158.8 92.7) (end 158.8 105.66) (width 0.2) (layer "F.Cu") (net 1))
 (segment (start 153.536827 134.010481) (end 154.210481 133.336827) (width 0.2) (layer "F.Cu") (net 1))
 (segment (start 143 93.9) (end 145.5 91.4) (width 0.2) (layer "F.Cu") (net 1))
 (segment (start 132.35 88.46) (end 132.35 110.42) (width 0.2) (layer "F.Cu") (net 1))
 (segment (start 109.54 88.42) (end 132.31 88.42) (width 0.2) (layer "F.Cu") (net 1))
 (segment (start 139.54 145.74) (end 145.314314 139.965686) (width 0.2) (layer "F.Cu") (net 1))
 (segment (start 132.35 88.46) (end 137.56 88.46) (width 0.2) (layer "F.Cu") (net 1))
 (segment (start 152.463173 136.036827) (end 153.536827 134.963173) (width 0.2) (layer "F.Cu") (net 1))
 (segment (start 156.316827 133.336827) (end 157.466827 134.486827) (width 0.2) (layer "F.Cu") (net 1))
 (segment (start 100.72 91.450101) (end 103.750101 88.42) (width 0.2) (layer "F.Cu") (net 1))
 (segment (start 145.503833 136.036827) (end 152.463173 136.036827) (width 0.2) (layer "F.Cu") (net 1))
 (segment (start 135.56 131.6) (end 143.18 131.6) (width 0.2) (layer "F.Cu") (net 1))
 (segment (start 158.8 105.66) (end 154.04 110.42) (width 0.2) (layer "F.Cu") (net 1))
 (segment (start 132.31 88.42) (end 132.35 88.46) (width 0.2) (layer "F.Cu") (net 1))
 (segment (start 154.210481 133.336827) (end 156.316827 133.336827) (width 0.2) (layer "F.Cu") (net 1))
 (segment (start 100.72 101.8) (end 100.72 91.450101) (width 0.2) (layer "F.Cu") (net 1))
 (segment (start 144.84066 139.492032) (end 144.84066 136.7) (width 0.2) (layer "F.Cu") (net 1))
 (segment (start 162 112.78) (end 162 95.9) (width 0.2) (layer "F.Cu") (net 1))
 (segment (start 137.56 88.46) (end 143 93.9) (width 0.2) (layer "F.Cu") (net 1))
 (segment (start 116.224365 131.6) (end 115.58 130.955635) (width 0.2) (layer "F.Cu") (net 11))
 (segment (start 115.58 130.955635) (end 115.58 127.603402) (width 0.2) (layer "F.Cu") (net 11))
 (segment (start 103.07 115.093402) (end 103.07 113.04) (width 0.2) (layer "F.Cu") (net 11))
 (segment (start 115.58 127.603402) (end 103.07 115.093402) (width 0.2) (layer "F.Cu") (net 11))
 (segment (start 119.22 130.5) (end 118.12 131.6) (width 0.2) (layer "F.Cu") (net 11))
 (segment (start 118.12 131.6) (end 116.224365 131.6) (width 0.2) (layer "F.Cu") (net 11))
 (segment (start 133.547308 136.3) (end 133 136.3) (width 0.2) (layer "F.Cu") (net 24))
 (segment (start 152.386827 134.486827) (end 151.236827 135.636827) (width 0.2) (layer "F.Cu") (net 24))
 (segment (start 151.236827 135.636827) (end 134.210481 135.636827) (width 0.2) (layer "F.Cu") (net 24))
 (segment (start 133 139.58) (end 126.84 145.74) (width 0.2) (layer "F.Cu") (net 24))
 (segment (start 134.210481 135.636827) (end 133.547308 136.3) (width 0.2) (layer "F.Cu") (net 24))
 (segment (start 133 136.3) (end 133 139.58) (width 0.2) (layer "F.Cu") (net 24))
 (segment (start 126.84 130.5) (end 143.800101 113.539899) (width 0.2) (layer "F.Cu") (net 6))
 (segment (start 146.29 113.539899) (end 147.110101 114.36) (width 0.2) (layer "F.Cu") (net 6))
 (segment (start 152.64 101.26) (end 157.5 96.4) (width 0.2) (layer "F.Cu") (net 6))
 (segment (start 143.800101 113.539899) (end 146.29 113.539899) (width 0.2) (layer "F.Cu") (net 6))
 (segment (start 147.110101 114.36) (end 148.269899 114.36) (width 0.2) (layer "F.Cu") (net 6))
 (segment (start 152.64 109.989899) (end 152.64 101.26) (width 0.2) (layer "F.Cu") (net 6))
 (segment (start 148.269899 114.36) (end 152.64 109.989899) (width 0.2) (layer "F.Cu") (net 6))
 (segment (start 145.433173 143.5) (end 145.913654 143.5) (width 0.2) (layer "F.Cu") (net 17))
 (segment (start 143.5 146.84) (end 110.16 146.84) (width 0.2) (layer "F.Cu") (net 17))
 (segment (start 110.16 146.84) (end 109.06 145.74) (width 0.2) (layer "F.Cu") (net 17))
 (segment (start 145.433173 143.5) (end 145.433173 144.906827) (width 0.2) (layer "F.Cu") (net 17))
 (segment (start 145.913654 143.5) (end 154.926827 134.486827) (width 0.2) (layer "F.Cu") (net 17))
 (segment (start 145.433173 144.906827) (end 143.5 146.84) (width 0.2) (layer "F.Cu") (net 17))
 (segment (start 128.28 131.6) (end 123.844365 131.6) (width 0.2) (layer "F.Cu") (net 5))
 (segment (start 123.2 130.955635) (end 123.2 130.044365) (width 0.2) (layer "F.Cu") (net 5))
 (segment (start 123.844365 131.6) (end 123.2 130.955635) (width 0.2) (layer "F.Cu") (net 5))
 (segment (start 123.2 130.044365) (end 143 110.244365) (width 0.2) (layer "F.Cu") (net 5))
 (segment (start 129.38 130.5) (end 128.28 131.6) (width 0.2) (layer "F.Cu") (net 5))
 (segment (start 143 110.244365) (end 143 96.4) (width 0.2) (layer "F.Cu") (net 5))
 (segment (start 124.3 130.5) (end 141.84 112.96) (width 0.2) (layer "F.Cu") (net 9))
 (segment (start 141.84 112.96) (end 147.69 112.96) (width 0.2) (layer "F.Cu") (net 9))
 (segment (start 149.846827 134.486827) (end 132.5 134.486827) (width 0.2) (layer "F.Cu") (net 23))
 (segment (start 132.5 134.486827) (end 131.836827 135.15) (width 0.2) (layer "F.Cu") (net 23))
 (segment (start 131.624314 138.415686) (end 124.3 145.74) (width 0.2) (layer "F.Cu") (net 23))
 (segment (start 131.15066 135.15) (end 131.836827 135.15) (width 0.2) (layer "F.Cu") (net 23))
 (segment (start 131.15066 135.15) (end 131.15066 137.942032) (width 0.2) (layer "F.Cu") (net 23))
 (segment (start 131.15066 137.942032) (end 131.624314 138.415686) (width 0.2) (layer "F.Cu") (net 23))
 (segment (start 129.435635 132) (end 121.704365 132) (width 0.2) (layer "F.Cu") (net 3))
 (segment (start 121.704365 132) (end 120.66 130.955635) (width 0.2) (layer "F.Cu") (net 3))
 (segment (start 120.66 99.307056) (end 126 93.967056) (width 0.2) (layer "F.Cu") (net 3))
 (segment (start 130.48 130.955635) (end 129.435635 132) (width 0.2) (layer "F.Cu") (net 3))
 (segment (start 130.48 127.425686) (end 130.48 130.955635) (width 0.2) (layer "F.Cu") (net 3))
 (segment (start 126 93.967056) (end 126 91) (width 0.2) (layer "F.Cu") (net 3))
 (segment (start 136.465686 127.425686) (end 130.48 127.425686) (width 0.2) (layer "F.Cu") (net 3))
 (segment (start 139.54 130.5) (end 136.465686 127.425686) (width 0.2) (layer "F.Cu") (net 3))
 (segment (start 120.66 130.955635) (end 120.66 99.307056) (width 0.2) (layer "F.Cu") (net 3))
 (segment (start 116.68 106.562944) (end 103.19 93.072944) (width 0.2) (layer "F.Cu") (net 2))
 (segment (start 116.68 130.5) (end 116.68 106.562944) (width 0.2) (layer "F.Cu") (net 2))
 (segment (start 103.19 93.072944) (end 103.19 90.96) (width 0.2) (layer "F.Cu") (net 2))
 (segment (start 163.9 95.961522) (end 158.038478 90.1) (width 0.2) (layer "F.Cu") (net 4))
 (segment (start 158.038478 90.1) (end 144.3 90.1) (width 0.2) (layer "F.Cu") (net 4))
 (segment (start 135.163173 132.336827) (end 158.5 132.336827) (width 0.2) (layer "F.Cu") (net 4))
 (segment (start 158.5 132.336827) (end 163.9 126.936827) (width 0.2) (layer "F.Cu") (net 4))
 (segment (start 163.9 126.936827) (end 163.9 95.961522) (width 0.2) (layer "F.Cu") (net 4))
 (segment (start 134.5 133) (end 135.163173 132.336827) (width 0.2) (layer "F.Cu") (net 4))
 (segment (start 134.42 133) (end 134.5 133) (width 0.2) (layer "F.Cu") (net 4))
 (segment (start 144.3 90.1) (end 143 91.4) (width 0.2) (layer "F.Cu") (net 4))
 (segment (start 131.92 130.5) (end 134.42 133) (width 0.2) (layer "F.Cu") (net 4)))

